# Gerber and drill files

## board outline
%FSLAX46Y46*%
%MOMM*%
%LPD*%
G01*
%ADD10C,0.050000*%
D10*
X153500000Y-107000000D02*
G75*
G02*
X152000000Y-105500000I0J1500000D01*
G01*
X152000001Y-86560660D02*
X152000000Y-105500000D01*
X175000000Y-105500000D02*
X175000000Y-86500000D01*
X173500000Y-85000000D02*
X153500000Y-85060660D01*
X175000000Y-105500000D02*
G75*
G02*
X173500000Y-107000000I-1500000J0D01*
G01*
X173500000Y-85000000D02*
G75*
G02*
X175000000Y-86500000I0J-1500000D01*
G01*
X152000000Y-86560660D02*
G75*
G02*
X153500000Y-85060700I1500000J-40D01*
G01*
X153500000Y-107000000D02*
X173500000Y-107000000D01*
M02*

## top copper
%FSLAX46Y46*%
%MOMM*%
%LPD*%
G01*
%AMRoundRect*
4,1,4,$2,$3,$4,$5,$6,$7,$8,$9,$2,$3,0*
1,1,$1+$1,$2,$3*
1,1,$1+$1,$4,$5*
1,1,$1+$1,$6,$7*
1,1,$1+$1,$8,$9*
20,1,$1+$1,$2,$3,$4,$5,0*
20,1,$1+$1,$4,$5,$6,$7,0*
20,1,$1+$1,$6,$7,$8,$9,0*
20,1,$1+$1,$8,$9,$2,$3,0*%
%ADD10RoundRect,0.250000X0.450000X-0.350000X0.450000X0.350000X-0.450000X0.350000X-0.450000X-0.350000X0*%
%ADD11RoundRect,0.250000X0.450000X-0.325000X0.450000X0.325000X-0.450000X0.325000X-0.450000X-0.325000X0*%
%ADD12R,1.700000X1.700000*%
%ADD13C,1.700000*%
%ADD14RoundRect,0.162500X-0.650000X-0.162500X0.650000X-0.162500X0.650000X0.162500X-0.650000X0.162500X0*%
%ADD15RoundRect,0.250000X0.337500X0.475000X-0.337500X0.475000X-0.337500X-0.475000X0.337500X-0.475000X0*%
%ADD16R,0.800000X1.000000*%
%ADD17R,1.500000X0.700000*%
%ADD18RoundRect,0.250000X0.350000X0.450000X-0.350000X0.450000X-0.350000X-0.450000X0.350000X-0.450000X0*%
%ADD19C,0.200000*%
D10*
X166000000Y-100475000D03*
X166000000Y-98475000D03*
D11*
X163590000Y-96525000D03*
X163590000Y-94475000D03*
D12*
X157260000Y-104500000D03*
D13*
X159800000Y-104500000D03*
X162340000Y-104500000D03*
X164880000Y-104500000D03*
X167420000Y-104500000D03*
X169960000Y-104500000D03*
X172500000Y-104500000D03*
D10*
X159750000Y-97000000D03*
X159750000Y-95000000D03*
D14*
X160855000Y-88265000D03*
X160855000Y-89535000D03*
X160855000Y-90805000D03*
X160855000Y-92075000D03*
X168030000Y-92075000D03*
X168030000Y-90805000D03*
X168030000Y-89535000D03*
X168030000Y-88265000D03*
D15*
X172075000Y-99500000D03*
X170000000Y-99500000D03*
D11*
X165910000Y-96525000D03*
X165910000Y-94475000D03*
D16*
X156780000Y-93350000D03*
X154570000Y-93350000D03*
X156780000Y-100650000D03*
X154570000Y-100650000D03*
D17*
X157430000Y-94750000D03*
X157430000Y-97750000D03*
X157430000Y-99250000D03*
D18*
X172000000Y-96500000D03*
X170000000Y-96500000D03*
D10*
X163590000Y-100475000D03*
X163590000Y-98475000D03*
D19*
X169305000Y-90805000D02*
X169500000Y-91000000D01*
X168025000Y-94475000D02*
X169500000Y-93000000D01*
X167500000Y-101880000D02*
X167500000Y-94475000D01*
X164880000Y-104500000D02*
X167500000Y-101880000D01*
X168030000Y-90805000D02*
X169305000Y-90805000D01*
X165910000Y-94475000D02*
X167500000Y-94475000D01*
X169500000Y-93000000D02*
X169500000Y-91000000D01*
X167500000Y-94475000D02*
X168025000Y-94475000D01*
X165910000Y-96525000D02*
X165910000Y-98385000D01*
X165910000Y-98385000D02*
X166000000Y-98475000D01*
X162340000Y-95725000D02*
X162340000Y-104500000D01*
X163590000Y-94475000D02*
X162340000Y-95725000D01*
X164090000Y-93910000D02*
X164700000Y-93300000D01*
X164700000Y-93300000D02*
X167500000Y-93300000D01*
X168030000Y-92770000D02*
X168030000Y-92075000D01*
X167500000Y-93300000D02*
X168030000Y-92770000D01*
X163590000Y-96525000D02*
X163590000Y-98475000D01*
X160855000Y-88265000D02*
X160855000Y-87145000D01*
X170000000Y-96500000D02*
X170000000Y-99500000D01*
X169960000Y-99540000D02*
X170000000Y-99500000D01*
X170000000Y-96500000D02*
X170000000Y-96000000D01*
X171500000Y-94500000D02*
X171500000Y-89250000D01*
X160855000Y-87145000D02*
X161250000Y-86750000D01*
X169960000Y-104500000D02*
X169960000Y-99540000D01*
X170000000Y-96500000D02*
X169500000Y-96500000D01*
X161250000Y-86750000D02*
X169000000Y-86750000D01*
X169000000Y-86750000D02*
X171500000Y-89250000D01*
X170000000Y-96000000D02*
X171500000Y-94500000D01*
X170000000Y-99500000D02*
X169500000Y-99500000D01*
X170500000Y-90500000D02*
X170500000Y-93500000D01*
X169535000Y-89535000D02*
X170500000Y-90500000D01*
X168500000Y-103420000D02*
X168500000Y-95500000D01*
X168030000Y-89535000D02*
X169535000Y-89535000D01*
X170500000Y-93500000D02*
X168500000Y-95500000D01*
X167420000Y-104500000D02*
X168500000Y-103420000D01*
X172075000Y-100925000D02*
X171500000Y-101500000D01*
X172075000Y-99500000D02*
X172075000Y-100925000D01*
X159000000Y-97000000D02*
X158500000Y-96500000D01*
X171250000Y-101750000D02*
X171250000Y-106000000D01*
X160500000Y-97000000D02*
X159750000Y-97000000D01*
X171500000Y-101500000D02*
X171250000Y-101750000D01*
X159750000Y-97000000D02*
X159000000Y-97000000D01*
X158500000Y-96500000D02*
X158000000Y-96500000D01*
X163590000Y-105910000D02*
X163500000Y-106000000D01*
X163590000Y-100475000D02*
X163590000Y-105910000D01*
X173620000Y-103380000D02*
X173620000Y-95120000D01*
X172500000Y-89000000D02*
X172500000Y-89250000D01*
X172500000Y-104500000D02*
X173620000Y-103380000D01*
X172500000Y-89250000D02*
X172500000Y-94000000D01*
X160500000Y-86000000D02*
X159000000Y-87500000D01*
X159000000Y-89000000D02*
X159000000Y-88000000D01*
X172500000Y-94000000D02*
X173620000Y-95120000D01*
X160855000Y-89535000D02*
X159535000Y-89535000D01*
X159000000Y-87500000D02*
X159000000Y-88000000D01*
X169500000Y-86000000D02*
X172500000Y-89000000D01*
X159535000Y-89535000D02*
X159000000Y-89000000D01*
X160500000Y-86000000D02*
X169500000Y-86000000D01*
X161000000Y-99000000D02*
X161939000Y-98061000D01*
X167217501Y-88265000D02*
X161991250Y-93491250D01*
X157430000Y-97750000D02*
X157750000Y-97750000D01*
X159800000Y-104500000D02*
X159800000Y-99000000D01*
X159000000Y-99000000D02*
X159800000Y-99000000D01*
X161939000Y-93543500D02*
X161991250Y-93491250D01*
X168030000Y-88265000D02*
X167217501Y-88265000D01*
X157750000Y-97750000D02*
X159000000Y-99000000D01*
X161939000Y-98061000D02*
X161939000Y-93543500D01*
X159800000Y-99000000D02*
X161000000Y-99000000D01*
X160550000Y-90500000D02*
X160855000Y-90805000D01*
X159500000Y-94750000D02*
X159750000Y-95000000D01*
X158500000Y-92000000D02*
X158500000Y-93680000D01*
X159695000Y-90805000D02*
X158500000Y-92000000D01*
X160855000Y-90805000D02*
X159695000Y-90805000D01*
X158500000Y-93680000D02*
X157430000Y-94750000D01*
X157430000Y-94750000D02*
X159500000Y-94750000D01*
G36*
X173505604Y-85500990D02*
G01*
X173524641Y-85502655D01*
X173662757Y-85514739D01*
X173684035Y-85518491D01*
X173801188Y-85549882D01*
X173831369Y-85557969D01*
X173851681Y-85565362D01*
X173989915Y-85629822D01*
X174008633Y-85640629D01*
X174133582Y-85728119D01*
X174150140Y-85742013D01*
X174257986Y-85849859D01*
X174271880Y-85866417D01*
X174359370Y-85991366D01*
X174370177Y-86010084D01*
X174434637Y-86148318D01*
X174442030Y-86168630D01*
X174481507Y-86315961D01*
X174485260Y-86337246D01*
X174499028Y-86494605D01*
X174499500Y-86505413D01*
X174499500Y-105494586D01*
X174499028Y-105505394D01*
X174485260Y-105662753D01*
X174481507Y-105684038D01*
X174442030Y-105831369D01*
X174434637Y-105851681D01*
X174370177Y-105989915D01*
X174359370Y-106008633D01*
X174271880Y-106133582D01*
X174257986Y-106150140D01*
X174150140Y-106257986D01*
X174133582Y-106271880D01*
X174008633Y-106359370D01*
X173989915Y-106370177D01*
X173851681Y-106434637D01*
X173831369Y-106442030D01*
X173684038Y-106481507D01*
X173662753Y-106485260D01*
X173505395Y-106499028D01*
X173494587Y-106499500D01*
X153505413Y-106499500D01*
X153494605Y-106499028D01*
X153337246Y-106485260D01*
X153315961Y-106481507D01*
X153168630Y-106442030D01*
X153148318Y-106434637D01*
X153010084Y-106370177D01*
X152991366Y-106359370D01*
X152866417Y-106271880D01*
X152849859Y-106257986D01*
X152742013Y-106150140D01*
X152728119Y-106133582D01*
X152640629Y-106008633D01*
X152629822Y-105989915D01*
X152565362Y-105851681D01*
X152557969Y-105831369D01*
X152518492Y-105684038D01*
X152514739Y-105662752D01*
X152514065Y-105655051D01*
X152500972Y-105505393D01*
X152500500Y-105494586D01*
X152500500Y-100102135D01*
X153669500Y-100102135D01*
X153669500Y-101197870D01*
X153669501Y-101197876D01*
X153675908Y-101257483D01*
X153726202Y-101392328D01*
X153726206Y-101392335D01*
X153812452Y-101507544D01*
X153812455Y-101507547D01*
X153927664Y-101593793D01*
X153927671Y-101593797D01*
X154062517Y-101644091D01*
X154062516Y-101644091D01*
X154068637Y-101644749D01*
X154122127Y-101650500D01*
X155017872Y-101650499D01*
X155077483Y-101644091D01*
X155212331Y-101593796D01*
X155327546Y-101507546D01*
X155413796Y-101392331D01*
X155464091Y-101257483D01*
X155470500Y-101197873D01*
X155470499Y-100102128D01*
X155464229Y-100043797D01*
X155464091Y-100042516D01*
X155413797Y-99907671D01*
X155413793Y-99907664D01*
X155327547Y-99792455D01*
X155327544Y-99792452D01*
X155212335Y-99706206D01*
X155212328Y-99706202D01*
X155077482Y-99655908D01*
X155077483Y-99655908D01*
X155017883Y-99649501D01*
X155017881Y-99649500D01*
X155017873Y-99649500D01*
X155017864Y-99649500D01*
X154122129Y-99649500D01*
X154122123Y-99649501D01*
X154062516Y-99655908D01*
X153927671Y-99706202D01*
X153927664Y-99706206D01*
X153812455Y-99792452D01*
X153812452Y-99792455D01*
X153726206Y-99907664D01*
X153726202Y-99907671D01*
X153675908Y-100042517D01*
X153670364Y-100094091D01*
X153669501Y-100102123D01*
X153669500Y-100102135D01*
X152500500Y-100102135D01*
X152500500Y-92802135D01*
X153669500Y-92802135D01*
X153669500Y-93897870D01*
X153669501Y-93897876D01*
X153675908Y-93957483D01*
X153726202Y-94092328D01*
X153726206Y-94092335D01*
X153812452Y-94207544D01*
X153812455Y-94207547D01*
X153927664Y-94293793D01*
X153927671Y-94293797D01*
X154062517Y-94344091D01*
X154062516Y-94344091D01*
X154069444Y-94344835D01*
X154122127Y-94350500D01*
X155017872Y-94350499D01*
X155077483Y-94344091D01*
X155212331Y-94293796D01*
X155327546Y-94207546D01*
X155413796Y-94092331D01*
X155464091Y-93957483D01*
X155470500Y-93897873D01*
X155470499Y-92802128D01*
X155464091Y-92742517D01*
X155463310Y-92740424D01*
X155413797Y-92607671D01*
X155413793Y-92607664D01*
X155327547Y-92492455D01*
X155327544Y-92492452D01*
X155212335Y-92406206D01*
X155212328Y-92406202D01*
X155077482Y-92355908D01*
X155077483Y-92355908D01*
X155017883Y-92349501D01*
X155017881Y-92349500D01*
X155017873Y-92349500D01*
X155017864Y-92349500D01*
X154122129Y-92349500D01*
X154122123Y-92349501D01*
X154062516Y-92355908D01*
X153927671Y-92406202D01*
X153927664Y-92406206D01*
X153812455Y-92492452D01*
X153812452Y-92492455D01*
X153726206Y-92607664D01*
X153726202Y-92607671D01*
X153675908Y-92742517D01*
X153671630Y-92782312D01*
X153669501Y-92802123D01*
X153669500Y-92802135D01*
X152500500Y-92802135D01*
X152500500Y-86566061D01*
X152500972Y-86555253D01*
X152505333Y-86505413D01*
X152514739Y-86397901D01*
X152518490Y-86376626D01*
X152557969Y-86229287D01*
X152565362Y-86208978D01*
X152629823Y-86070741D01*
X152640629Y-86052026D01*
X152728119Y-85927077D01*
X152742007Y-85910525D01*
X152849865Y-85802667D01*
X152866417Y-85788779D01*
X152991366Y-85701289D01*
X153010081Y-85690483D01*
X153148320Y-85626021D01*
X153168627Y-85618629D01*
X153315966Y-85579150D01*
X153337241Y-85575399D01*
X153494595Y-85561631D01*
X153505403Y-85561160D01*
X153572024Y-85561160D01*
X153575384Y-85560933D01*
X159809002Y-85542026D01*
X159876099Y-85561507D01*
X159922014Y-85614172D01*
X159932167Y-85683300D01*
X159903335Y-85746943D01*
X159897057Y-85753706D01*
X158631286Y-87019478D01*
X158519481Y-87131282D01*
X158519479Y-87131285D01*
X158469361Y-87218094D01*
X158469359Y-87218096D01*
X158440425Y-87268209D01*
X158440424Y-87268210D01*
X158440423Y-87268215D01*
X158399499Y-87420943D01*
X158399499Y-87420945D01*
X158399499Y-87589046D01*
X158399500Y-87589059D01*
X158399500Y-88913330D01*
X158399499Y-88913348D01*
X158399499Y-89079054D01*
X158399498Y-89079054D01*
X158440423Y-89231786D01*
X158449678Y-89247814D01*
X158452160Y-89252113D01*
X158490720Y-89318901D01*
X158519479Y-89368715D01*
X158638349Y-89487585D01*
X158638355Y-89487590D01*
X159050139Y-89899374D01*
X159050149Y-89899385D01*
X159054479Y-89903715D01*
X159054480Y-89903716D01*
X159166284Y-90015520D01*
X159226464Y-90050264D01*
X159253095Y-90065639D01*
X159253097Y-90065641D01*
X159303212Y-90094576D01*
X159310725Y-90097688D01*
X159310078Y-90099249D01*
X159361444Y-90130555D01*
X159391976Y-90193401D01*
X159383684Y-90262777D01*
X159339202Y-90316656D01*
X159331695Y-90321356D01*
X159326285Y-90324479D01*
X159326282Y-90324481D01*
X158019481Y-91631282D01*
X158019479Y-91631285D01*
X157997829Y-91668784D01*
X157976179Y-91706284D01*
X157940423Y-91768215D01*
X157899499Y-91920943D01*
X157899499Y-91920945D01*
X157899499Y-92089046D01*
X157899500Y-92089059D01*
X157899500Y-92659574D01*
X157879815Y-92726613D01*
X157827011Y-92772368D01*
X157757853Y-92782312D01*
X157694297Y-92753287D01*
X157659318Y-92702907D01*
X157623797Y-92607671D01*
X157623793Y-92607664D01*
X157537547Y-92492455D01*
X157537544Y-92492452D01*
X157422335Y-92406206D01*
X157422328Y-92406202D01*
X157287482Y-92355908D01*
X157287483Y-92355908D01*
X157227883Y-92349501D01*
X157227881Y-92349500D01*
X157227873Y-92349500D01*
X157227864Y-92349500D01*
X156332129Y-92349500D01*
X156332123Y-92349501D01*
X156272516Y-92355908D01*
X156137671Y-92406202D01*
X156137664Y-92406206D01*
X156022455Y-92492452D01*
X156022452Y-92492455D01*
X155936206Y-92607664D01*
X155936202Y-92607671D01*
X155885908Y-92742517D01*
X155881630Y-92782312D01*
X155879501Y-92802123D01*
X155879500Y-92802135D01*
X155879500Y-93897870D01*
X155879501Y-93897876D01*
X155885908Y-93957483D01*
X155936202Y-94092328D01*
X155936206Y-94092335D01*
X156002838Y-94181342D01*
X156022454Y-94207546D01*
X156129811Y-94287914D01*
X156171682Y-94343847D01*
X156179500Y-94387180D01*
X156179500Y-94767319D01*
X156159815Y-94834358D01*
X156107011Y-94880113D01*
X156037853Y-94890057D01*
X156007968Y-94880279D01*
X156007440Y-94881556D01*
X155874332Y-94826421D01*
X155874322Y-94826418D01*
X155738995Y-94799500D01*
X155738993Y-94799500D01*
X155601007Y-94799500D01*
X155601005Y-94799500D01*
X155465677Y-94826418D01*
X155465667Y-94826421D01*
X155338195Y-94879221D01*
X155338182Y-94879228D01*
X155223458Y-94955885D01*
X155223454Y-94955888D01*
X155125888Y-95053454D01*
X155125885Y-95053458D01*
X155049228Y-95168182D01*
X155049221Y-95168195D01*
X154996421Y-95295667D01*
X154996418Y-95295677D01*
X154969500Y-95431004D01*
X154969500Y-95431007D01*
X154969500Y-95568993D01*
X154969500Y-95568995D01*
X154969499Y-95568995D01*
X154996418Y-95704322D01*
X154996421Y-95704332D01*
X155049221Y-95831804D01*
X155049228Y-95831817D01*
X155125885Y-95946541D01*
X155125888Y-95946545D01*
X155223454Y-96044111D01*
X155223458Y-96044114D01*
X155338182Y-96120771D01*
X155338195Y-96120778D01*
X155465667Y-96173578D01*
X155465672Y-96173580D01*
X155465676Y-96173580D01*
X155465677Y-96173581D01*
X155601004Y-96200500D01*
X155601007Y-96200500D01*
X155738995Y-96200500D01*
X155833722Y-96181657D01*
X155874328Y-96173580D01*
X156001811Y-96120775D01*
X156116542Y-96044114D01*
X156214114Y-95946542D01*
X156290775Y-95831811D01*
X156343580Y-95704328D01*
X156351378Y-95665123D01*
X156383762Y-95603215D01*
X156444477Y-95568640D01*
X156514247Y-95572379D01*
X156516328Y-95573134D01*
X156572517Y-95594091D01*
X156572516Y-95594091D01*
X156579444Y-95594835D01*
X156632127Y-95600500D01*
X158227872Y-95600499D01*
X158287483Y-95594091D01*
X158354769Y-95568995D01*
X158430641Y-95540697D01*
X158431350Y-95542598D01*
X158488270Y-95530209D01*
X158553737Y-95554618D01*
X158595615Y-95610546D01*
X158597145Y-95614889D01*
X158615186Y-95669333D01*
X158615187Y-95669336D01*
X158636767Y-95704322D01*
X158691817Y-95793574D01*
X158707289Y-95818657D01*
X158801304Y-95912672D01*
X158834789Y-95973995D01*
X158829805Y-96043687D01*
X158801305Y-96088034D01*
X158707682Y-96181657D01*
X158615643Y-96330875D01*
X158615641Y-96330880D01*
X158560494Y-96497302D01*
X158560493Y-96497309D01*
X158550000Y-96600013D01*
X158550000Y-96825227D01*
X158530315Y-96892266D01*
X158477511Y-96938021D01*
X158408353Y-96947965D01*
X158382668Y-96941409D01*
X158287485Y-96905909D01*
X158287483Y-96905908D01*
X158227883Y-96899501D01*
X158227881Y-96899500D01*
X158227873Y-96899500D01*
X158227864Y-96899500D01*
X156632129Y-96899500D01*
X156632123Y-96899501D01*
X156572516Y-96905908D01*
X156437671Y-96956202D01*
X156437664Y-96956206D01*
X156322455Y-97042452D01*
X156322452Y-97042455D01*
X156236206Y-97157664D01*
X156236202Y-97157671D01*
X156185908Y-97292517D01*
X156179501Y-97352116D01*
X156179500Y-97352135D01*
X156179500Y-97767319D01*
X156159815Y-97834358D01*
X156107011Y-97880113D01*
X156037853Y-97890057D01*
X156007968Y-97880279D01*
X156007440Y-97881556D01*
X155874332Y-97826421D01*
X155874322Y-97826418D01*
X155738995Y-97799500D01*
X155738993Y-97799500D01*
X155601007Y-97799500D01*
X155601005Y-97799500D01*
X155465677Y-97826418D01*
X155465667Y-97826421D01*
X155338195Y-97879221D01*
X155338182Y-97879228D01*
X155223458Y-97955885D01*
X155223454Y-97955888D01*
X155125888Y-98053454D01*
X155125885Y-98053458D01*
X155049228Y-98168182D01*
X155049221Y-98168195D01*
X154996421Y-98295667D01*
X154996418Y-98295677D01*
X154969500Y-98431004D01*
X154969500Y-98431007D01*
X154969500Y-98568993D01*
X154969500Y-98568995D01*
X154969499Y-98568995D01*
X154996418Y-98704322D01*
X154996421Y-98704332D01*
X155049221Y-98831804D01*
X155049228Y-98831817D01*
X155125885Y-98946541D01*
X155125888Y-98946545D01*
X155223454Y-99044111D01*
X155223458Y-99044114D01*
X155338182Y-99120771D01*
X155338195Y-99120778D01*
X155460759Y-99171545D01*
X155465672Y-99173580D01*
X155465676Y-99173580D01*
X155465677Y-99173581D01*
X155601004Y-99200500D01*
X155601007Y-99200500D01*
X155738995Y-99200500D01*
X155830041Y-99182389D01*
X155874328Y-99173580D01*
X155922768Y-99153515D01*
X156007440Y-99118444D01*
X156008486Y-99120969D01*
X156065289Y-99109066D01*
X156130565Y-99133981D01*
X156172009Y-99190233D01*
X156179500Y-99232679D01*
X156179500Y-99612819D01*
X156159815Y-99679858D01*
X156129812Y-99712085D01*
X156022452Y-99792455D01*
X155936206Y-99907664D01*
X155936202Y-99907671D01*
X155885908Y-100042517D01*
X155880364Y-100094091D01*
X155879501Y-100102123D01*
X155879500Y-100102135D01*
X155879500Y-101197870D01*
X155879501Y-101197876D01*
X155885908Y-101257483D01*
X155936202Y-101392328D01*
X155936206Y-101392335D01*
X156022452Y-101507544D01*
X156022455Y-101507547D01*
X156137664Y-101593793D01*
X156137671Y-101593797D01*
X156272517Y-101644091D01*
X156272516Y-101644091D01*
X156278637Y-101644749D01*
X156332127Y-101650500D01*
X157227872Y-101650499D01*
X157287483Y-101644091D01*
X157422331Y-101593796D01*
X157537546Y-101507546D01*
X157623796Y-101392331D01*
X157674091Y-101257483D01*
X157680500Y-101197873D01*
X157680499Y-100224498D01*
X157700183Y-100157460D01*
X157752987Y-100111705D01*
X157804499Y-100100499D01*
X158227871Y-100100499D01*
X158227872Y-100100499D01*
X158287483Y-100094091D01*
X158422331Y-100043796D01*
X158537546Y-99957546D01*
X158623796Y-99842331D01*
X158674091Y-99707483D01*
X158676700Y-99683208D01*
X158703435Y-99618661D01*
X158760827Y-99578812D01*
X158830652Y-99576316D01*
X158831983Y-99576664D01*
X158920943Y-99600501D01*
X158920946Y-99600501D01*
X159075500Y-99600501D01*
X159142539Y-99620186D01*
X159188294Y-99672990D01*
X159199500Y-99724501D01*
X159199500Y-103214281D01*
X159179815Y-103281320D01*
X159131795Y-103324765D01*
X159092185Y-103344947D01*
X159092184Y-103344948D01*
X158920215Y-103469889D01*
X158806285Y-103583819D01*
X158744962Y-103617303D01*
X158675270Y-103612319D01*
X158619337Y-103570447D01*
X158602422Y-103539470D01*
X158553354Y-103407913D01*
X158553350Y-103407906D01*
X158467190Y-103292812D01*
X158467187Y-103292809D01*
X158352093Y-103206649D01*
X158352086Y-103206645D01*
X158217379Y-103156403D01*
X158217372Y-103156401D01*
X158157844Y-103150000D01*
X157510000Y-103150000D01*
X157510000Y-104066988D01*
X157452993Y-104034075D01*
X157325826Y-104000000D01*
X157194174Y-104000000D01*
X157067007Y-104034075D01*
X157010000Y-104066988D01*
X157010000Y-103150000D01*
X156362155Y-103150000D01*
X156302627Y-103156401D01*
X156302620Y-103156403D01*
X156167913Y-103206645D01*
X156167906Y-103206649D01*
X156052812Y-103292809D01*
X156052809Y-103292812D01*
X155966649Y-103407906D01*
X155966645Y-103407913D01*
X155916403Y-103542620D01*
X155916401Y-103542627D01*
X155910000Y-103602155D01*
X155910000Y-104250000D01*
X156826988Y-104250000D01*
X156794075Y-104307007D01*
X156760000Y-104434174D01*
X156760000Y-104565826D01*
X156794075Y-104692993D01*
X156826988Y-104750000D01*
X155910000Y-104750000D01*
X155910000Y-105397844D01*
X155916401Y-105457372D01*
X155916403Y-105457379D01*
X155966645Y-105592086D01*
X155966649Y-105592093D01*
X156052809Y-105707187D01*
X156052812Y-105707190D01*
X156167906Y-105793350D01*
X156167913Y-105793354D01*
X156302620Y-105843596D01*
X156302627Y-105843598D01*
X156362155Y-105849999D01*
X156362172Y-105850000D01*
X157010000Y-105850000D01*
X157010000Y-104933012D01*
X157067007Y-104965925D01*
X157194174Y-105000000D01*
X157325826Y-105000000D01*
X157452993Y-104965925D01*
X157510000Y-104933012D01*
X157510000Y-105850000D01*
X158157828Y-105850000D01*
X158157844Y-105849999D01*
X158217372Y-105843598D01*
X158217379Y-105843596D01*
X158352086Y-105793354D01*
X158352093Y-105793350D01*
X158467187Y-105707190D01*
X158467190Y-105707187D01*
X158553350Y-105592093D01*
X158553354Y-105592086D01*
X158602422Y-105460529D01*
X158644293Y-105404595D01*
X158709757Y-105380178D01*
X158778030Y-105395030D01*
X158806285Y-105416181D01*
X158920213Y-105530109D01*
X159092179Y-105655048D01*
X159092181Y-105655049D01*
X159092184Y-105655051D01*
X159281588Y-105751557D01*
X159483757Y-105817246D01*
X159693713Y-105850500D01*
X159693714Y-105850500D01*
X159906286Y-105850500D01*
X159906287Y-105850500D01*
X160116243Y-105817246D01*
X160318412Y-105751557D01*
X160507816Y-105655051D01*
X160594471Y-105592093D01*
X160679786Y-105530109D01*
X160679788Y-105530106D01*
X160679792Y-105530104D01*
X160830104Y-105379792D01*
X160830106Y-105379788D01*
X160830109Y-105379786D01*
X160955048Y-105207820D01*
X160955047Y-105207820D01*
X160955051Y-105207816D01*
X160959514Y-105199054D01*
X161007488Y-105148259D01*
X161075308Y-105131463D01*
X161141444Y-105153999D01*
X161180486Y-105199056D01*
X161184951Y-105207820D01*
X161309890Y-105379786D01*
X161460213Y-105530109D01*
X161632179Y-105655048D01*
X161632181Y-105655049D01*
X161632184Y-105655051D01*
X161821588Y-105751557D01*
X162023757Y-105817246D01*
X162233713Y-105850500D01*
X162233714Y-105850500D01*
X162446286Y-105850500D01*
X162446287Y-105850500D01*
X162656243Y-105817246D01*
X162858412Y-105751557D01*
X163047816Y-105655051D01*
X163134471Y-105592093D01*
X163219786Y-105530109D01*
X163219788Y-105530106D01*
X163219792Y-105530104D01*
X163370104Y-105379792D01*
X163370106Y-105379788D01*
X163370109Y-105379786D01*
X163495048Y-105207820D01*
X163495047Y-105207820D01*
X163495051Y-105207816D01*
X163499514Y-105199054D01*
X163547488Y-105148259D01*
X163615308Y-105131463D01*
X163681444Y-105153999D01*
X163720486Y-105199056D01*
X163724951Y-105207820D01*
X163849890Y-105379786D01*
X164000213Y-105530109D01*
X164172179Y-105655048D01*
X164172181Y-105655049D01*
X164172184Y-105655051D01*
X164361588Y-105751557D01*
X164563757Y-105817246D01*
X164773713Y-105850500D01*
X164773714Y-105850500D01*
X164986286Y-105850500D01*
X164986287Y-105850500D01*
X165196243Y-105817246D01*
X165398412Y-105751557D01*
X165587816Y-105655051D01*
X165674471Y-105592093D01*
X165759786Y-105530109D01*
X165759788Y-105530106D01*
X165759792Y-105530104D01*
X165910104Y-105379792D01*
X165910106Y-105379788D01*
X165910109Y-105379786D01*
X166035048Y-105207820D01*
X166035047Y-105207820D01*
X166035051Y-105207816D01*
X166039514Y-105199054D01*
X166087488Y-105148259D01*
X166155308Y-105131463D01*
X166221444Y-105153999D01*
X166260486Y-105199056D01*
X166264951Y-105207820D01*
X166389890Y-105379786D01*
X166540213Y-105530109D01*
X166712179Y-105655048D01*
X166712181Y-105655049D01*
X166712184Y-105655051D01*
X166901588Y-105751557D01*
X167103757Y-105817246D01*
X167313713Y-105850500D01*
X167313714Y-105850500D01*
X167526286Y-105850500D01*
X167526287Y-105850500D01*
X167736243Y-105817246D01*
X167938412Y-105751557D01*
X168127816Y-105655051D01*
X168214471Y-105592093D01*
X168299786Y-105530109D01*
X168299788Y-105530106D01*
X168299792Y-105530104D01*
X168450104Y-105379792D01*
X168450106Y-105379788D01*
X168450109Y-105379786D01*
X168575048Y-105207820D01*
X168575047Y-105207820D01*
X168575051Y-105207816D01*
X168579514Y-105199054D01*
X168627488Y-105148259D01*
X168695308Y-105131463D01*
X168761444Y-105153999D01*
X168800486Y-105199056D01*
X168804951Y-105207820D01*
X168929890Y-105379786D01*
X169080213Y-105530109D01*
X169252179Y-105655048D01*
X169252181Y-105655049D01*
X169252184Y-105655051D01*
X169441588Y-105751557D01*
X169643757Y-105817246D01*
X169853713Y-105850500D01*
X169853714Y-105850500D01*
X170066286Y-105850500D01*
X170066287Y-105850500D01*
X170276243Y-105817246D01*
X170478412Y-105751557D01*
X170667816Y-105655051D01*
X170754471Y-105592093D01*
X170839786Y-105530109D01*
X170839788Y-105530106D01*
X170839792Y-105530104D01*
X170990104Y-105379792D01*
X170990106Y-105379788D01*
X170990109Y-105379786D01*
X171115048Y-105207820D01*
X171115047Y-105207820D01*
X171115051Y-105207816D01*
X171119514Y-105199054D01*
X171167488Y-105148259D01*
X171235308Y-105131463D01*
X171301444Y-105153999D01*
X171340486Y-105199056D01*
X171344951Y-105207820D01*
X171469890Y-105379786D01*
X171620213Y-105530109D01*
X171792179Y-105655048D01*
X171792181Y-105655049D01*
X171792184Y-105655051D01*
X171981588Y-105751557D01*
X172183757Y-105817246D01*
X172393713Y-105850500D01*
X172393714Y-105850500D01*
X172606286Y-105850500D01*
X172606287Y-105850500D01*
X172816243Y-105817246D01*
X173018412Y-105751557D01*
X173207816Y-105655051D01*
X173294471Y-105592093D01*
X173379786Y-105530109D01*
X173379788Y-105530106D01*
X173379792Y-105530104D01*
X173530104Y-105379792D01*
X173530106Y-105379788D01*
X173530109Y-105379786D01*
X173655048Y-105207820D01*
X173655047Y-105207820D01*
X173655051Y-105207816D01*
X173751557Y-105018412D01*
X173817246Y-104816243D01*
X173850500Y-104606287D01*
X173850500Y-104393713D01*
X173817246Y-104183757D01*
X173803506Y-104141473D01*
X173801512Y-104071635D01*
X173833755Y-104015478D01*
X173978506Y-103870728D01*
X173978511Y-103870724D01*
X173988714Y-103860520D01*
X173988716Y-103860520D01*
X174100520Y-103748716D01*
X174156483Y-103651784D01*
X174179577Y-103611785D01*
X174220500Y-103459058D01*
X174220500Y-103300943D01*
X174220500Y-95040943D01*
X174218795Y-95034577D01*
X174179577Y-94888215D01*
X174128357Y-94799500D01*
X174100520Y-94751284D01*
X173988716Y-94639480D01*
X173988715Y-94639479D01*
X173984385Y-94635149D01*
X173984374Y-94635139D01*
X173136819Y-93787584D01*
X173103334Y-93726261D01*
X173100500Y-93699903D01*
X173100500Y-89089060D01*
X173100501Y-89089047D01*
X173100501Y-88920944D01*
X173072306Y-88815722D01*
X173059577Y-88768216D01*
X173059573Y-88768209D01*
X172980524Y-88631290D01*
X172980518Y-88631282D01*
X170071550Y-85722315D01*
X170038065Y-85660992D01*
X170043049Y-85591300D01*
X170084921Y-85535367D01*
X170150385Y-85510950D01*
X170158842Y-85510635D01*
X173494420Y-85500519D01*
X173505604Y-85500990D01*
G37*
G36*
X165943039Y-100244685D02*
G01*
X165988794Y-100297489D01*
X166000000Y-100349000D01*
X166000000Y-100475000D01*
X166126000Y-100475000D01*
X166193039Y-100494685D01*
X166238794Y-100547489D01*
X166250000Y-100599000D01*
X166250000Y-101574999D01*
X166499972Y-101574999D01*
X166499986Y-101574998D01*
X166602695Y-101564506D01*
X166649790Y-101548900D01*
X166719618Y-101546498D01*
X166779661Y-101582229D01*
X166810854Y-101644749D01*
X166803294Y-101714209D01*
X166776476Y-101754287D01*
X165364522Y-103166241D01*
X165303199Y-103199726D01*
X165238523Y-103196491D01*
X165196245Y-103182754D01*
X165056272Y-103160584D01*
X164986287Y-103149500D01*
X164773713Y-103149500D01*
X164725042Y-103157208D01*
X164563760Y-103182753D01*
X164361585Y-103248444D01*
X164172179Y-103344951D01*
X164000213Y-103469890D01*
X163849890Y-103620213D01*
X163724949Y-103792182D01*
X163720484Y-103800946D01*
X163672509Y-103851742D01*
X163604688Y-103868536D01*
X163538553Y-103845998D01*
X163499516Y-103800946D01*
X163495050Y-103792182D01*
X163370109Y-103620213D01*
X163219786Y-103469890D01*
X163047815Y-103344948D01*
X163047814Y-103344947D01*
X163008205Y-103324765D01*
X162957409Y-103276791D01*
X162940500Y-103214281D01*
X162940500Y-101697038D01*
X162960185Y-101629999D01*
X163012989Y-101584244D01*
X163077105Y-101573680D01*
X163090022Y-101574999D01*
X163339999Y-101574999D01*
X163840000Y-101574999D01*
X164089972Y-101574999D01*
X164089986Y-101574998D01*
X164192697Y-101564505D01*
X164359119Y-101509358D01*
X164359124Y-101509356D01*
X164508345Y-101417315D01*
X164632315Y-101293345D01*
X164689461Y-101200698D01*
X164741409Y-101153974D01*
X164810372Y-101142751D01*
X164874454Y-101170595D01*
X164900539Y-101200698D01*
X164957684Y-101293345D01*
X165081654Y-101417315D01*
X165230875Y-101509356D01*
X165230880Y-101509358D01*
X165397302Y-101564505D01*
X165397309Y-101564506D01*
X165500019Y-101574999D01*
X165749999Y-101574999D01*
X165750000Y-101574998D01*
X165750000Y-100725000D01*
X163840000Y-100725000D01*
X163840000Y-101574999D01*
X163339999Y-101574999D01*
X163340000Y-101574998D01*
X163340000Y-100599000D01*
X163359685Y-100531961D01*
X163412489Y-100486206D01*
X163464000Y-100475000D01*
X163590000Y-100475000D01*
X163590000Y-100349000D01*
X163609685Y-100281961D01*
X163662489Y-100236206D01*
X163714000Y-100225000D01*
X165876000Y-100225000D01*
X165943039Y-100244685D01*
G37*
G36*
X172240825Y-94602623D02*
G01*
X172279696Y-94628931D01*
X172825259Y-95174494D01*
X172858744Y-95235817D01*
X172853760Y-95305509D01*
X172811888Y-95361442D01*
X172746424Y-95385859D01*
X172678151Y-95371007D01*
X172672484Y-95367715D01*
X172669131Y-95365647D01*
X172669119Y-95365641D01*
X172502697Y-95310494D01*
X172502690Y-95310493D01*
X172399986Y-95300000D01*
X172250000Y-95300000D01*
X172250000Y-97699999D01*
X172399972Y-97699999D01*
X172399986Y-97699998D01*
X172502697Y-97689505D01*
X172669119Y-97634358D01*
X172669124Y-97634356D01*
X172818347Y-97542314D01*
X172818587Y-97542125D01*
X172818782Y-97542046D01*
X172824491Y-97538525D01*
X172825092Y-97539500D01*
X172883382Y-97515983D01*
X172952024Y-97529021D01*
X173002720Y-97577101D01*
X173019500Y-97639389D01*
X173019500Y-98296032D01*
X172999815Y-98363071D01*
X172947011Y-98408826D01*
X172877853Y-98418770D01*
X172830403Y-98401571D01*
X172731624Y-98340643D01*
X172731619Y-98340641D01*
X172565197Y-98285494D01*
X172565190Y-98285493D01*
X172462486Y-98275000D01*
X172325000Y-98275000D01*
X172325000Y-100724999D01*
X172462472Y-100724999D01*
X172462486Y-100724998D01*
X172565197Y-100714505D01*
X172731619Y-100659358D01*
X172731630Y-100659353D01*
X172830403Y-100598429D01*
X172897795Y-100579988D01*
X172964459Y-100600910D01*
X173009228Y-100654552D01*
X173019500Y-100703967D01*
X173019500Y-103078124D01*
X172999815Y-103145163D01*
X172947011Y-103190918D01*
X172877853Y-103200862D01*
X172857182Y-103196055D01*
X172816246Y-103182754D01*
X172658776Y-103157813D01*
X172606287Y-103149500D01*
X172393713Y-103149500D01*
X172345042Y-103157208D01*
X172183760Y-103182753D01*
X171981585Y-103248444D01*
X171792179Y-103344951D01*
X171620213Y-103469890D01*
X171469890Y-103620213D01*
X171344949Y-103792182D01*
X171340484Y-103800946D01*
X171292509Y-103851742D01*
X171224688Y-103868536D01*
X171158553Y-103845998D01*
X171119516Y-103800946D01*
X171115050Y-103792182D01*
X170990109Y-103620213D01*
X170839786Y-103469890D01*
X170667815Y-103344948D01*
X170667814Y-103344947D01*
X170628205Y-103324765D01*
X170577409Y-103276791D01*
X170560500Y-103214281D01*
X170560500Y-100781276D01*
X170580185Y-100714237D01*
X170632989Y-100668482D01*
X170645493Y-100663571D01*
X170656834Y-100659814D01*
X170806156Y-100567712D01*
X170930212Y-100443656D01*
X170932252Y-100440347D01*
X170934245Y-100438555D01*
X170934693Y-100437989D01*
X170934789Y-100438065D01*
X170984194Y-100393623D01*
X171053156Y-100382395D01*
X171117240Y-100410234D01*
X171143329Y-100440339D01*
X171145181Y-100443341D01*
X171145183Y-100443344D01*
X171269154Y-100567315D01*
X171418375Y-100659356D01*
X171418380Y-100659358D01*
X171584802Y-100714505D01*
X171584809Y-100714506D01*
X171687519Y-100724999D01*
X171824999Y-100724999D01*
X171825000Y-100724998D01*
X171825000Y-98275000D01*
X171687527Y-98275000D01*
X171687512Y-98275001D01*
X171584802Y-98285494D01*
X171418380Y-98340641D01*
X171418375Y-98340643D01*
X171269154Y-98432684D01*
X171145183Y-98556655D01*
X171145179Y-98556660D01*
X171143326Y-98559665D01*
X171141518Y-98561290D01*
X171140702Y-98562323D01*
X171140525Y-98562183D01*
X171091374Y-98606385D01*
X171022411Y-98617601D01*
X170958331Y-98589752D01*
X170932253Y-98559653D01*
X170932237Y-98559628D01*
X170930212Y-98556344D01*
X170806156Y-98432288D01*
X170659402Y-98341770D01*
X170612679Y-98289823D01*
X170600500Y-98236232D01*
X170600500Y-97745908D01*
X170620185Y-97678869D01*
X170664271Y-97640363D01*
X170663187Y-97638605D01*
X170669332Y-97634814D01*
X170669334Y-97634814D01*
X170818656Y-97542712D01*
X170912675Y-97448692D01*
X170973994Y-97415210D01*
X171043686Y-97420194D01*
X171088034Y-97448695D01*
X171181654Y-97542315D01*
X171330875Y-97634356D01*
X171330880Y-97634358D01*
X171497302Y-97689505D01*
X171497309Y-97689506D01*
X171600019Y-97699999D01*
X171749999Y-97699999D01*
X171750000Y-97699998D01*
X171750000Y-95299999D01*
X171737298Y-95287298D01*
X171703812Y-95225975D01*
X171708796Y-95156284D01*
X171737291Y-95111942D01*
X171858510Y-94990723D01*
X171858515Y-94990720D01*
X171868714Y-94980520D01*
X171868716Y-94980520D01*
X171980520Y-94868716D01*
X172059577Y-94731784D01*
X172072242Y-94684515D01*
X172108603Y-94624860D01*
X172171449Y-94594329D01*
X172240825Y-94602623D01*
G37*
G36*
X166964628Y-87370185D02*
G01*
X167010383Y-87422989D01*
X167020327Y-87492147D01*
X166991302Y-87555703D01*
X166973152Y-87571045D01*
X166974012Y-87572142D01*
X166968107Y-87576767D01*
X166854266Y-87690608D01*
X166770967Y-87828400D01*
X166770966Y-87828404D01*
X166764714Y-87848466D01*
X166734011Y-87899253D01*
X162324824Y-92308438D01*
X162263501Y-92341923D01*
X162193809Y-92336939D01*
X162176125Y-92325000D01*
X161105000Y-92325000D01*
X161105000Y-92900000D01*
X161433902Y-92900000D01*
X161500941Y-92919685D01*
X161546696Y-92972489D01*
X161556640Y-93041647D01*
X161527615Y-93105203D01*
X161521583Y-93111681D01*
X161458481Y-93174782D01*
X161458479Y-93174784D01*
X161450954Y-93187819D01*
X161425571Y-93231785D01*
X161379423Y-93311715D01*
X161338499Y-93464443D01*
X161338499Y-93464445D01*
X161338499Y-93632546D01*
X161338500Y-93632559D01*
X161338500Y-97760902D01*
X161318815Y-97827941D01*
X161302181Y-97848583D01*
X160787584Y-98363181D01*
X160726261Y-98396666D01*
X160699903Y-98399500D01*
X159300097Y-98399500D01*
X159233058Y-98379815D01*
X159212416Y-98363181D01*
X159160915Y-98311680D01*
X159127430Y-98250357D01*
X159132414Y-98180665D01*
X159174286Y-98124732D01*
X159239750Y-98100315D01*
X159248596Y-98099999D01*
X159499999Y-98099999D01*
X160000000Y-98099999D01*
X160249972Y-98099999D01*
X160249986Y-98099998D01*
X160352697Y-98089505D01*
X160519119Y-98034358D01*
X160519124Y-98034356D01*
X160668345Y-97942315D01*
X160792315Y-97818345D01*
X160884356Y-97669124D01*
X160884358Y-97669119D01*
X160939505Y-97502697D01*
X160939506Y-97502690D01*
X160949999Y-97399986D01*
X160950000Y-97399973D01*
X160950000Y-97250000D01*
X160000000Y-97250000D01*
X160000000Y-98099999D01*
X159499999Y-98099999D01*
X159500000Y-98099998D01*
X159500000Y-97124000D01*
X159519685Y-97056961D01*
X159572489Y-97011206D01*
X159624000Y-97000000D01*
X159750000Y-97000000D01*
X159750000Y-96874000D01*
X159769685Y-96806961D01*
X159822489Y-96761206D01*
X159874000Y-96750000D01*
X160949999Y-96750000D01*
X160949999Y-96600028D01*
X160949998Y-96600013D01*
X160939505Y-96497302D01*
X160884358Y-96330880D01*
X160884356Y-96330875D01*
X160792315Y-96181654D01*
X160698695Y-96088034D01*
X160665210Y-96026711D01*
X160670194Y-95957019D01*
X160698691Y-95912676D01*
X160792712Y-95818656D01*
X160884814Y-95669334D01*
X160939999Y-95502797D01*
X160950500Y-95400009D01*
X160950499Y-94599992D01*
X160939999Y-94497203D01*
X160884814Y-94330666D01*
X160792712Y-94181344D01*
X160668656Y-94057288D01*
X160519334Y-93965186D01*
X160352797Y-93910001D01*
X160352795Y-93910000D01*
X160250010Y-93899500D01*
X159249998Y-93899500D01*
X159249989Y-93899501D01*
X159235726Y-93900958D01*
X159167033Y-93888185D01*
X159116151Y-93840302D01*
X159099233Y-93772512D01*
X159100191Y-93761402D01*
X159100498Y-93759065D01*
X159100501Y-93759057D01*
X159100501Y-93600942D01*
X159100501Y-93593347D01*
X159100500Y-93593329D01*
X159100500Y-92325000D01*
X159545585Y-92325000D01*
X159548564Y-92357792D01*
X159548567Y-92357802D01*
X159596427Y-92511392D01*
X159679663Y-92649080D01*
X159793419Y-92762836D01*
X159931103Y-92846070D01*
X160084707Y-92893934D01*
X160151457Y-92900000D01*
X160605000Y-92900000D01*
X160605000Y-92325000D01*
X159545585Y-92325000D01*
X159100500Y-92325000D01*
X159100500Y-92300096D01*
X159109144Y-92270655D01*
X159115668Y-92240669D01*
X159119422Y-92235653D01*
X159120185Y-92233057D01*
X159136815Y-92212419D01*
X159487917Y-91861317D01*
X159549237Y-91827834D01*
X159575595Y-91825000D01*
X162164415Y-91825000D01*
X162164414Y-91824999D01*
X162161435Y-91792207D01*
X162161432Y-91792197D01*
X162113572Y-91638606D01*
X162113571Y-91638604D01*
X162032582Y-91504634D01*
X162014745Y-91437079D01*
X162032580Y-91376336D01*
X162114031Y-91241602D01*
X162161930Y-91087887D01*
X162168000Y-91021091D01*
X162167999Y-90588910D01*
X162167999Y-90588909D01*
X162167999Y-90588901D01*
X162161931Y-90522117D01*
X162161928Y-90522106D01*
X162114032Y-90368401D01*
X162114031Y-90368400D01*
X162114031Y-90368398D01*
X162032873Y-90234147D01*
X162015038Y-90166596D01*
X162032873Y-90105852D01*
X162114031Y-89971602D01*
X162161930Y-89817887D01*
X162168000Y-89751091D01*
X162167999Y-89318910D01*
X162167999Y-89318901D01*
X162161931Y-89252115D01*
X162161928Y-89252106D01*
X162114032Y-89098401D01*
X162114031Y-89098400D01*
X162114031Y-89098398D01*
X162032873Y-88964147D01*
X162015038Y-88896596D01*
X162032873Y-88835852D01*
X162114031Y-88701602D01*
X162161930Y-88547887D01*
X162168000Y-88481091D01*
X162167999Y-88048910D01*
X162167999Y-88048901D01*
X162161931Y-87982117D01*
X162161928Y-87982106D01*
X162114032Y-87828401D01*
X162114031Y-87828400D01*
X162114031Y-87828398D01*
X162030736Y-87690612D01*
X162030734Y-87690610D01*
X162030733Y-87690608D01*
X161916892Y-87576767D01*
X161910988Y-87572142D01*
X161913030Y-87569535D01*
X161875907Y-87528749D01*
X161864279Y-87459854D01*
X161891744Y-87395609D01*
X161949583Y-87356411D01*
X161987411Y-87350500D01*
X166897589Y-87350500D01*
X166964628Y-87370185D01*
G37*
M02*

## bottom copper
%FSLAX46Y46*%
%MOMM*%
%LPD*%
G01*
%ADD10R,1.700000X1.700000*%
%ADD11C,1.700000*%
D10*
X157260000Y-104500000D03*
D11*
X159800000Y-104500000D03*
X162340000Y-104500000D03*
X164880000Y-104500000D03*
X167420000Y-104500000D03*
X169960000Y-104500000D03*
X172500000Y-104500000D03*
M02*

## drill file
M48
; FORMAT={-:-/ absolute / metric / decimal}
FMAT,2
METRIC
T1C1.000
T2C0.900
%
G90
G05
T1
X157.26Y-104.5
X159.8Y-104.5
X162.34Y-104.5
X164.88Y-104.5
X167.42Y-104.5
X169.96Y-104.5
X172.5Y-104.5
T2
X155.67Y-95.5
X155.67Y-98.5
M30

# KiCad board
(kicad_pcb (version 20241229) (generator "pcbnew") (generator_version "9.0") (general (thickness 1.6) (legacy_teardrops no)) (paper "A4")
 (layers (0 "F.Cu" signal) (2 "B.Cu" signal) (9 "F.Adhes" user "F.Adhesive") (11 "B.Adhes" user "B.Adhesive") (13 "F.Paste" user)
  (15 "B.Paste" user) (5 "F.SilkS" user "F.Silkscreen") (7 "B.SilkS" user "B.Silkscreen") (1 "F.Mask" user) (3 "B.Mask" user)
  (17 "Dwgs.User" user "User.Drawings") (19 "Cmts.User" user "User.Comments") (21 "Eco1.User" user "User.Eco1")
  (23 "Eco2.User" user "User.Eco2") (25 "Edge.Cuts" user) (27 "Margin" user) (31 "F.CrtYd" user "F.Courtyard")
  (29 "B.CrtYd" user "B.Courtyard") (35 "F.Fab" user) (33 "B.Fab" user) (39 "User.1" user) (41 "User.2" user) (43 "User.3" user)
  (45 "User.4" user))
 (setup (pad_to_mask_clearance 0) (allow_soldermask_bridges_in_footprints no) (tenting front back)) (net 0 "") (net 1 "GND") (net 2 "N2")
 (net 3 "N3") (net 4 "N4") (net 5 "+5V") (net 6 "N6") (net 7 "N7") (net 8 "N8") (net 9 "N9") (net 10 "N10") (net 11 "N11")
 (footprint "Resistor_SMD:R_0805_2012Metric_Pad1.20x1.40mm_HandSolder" (layer "F.Cu") (at 166 99.475 90)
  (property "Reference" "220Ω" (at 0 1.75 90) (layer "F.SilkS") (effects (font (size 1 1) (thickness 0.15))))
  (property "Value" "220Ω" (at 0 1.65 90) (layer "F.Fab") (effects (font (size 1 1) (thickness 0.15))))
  (pad "1" smd roundrect (at -1 0 90) (size 1.2 1.4) (layers "F.Cu" "F.Mask" "F.Paste") (roundrect_rratio 0.208333) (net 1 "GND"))
  (pad "2" smd roundrect (at 1 0 90) (size 1.2 1.4) (layers "F.Cu" "F.Mask" "F.Paste") (roundrect_rratio 0.208333) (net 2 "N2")))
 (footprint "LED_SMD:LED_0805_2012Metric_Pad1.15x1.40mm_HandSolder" (layer "F.Cu") (at 163.59 95.5 90)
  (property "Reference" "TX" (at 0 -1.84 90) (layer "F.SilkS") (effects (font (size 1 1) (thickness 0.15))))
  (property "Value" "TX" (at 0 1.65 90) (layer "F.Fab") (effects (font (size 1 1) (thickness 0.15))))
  (pad "1" smd roundrect (at -1.025 0 90) (size 1.15 1.4) (layers "F.Cu" "F.Mask" "F.Paste") (roundrect_rratio 0.217391) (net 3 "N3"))
  (pad "2" smd roundrect (at 1.025 0 90) (size 1.15 1.4) (layers "F.Cu" "F.Mask" "F.Paste") (roundrect_rratio 0.217391) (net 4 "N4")))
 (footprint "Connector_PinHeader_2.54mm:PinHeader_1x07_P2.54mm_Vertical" (layer "F.Cu") (at 157.26 104.5 90)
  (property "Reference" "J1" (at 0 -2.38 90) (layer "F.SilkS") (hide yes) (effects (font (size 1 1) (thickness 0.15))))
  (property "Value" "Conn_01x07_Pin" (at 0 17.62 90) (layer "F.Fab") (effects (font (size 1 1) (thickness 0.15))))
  (pad "1" thru_hole rect (at 0 0 90) (size 1.7 1.7) (drill 1) (layers "*.Cu" "*.Mask") (remove_unused_layers no) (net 1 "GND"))
  (pad "2" thru_hole circle (at 0 2.54 90) (size 1.7 1.7) (drill 1) (layers "*.Cu" "*.Mask") (remove_unused_layers no) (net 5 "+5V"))
  (pad "3" thru_hole circle (at 0 5.08 90) (size 1.7 1.7) (drill 1) (layers "*.Cu" "*.Mask") (remove_unused_layers no) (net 4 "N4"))
  (pad "4" thru_hole circle (at 0 7.62 90) (size 1.7 1.7) (drill 1) (layers "*.Cu" "*.Mask") (remove_unused_layers no) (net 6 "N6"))
  (pad "5" thru_hole circle (at 0 10.16 90) (size 1.7 1.7) (drill 1) (layers "*.Cu" "*.Mask") (remove_unused_layers no) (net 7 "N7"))
  (pad "6" thru_hole circle (at 0 12.7 90) (size 1.7 1.7) (drill 1) (layers "*.Cu" "*.Mask") (remove_unused_layers no) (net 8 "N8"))
  (pad "7" thru_hole circle (at 0 15.24 90) (size 1.7 1.7) (drill 1) (layers "*.Cu" "*.Mask") (remove_unused_layers no) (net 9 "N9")))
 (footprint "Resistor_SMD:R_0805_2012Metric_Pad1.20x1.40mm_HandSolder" (layer "F.Cu") (at 159.75 96 90)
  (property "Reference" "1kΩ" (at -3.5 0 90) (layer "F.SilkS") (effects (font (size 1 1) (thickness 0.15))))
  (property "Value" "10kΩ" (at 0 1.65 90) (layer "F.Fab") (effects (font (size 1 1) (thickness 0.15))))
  (pad "1" smd roundrect (at -1 0 90) (size 1.2 1.4) (layers "F.Cu" "F.Mask" "F.Paste") (roundrect_rratio 0.208333) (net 1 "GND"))
  (pad "2" smd roundrect (at 1 0 90) (size 1.2 1.4) (layers "F.Cu" "F.Mask" "F.Paste") (roundrect_rratio 0.208333) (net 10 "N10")))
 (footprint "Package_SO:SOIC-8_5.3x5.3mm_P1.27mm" (layer "F.Cu") (at 164.4425 90.17)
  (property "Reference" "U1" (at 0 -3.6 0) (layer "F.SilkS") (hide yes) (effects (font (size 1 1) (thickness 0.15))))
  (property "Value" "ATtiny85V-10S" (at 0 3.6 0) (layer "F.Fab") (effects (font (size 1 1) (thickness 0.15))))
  (pad "1" smd roundrect (at -3.5875 -1.905) (size 1.625 0.65) (layers "F.Cu" "F.Mask" "F.Paste") (roundrect_rratio 0.25) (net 8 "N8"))
  (pad "2" smd roundrect (at -3.5875 -0.635) (size 1.625 0.65) (layers "F.Cu" "F.Mask" "F.Paste") (roundrect_rratio 0.25) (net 9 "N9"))
  (pad "3" smd roundrect (at -3.5875 0.635) (size 1.625 0.65) (layers "F.Cu" "F.Mask" "F.Paste") (roundrect_rratio 0.25) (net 10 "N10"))
  (pad "4" smd roundrect (at -3.5875 1.905) (size 1.625 0.65) (layers "F.Cu" "F.Mask" "F.Paste") (roundrect_rratio 0.25) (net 1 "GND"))
  (pad "5" smd roundrect (at 3.5875 1.905) (size 1.625 0.65) (layers "F.Cu" "F.Mask" "F.Paste") (roundrect_rratio 0.25) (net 4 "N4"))
  (pad "6" smd roundrect (at 3.5875 0.635) (size 1.625 0.65) (layers "F.Cu" "F.Mask" "F.Paste") (roundrect_rratio 0.25) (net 6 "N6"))
  (pad "7" smd roundrect (at 3.5875 -0.635) (size 1.625 0.65) (layers "F.Cu" "F.Mask" "F.Paste") (roundrect_rratio 0.25) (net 7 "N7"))
  (pad "8" smd roundrect (at 3.5875 -1.905) (size 1.625 0.65) (layers "F.Cu" "F.Mask" "F.Paste") (roundrect_rratio 0.25) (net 5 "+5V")))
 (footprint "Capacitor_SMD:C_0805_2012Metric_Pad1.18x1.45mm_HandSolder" (layer "F.Cu") (at 171.0375 99.5 180)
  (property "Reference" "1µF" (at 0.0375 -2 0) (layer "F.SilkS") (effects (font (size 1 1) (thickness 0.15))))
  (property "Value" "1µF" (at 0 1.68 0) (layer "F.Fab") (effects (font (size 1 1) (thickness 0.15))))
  (pad "1" smd roundrect (at -1.0375 0 180) (size 1.175 1.45) (layers "F.Cu" "F.Mask" "F.Paste") (roundrect_rratio 0.212766) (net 1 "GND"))
  (pad "2" smd roundrect (at 1.0375 0 180) (size 1.175 1.45) (layers "F.Cu" "F.Mask" "F.Paste") (roundrect_rratio 0.212766) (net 8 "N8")))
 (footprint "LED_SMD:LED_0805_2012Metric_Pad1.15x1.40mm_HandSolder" (layer "F.Cu") (at 165.91 95.5 90)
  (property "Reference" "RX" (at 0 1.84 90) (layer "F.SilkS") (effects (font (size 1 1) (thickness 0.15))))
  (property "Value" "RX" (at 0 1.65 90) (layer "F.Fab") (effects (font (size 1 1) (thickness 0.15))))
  (pad "1" smd roundrect (at -1.025 0 90) (size 1.15 1.4) (layers "F.Cu" "F.Mask" "F.Paste") (roundrect_rratio 0.217391) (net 2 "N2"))
  (pad "2" smd roundrect (at 1.025 0 90) (size 1.15 1.4) (layers "F.Cu" "F.Mask" "F.Paste") (roundrect_rratio 0.217391) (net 6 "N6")))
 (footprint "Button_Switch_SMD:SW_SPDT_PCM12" (layer "F.Cu") (at 156 97 -90)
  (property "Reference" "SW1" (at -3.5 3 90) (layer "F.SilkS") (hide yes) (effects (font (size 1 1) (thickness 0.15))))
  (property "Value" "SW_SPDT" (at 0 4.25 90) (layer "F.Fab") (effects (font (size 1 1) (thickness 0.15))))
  (pad "" smd rect (at -3.65 -0.78 270) (size 1 0.8) (layers "F.Cu" "F.Mask" "F.Paste"))
  (pad "" smd rect (at -3.65 1.43 270) (size 1 0.8) (layers "F.Cu" "F.Mask" "F.Paste"))
  (pad "" np_thru_hole circle (at -1.5 0.33 270) (size 0.9 0.9) (drill 0.9) (layers "*.Cu" "*.Mask"))
  (pad "" np_thru_hole circle (at 1.5 0.33 270) (size 0.9 0.9) (drill 0.9) (layers "*.Cu" "*.Mask"))
  (pad "" smd rect (at 3.65 -0.78 270) (size 1 0.8) (layers "F.Cu" "F.Mask" "F.Paste"))
  (pad "" smd rect (at 3.65 1.43 270) (size 1 0.8) (layers "F.Cu" "F.Mask" "F.Paste"))
  (pad "1" smd rect (at -2.25 -1.43 270) (size 0.7 1.5) (layers "F.Cu" "F.Mask" "F.Paste") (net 10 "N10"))
  (pad "2" smd rect (at 0.75 -1.43 270) (size 0.7 1.5) (layers "F.Cu" "F.Mask" "F.Paste") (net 5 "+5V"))
  (pad "3" smd rect (at 2.25 -1.43 270) (size 0.7 1.5) (layers "F.Cu" "F.Mask" "F.Paste") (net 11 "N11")))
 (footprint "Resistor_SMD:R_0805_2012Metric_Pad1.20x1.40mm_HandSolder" (layer "F.Cu") (at 171 96.5 180)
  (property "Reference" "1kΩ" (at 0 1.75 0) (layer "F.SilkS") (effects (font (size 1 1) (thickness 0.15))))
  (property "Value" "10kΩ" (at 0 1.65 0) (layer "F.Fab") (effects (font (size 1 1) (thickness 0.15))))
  (pad "1" smd roundrect (at -1 0 180) (size 1.2 1.4) (layers "F.Cu" "F.Mask" "F.Paste") (roundrect_rratio 0.208333) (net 1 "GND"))
  (pad "2" smd roundrect (at 1 0 180) (size 1.2 1.4) (layers "F.Cu" "F.Mask" "F.Paste") (roundrect_rratio 0.208333) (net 8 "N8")))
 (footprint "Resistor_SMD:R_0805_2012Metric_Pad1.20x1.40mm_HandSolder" (layer "F.Cu") (at 163.59 99.475 90)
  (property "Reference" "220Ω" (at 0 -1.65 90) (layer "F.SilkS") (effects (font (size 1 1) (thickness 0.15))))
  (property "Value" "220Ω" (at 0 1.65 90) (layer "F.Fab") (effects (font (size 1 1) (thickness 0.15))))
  (pad "1" smd roundrect (at -1 0 90) (size 1.2 1.4) (layers "F.Cu" "F.Mask" "F.Paste") (roundrect_rratio 0.208333) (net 1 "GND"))
  (pad "2" smd roundrect (at 1 0 90) (size 1.2 1.4) (layers "F.Cu" "F.Mask" "F.Paste") (roundrect_rratio 0.208333) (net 3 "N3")))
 (gr_arc (start 153.5 107) (mid 152.43934 106.56066) (end 152 105.5) (stroke (width 0.05) (type default)) (layer "Edge.Cuts"))
 (gr_line (start 152.000001 86.56066) (end 152 105.5) (stroke (width 0.05) (type default)) (layer "Edge.Cuts"))
 (gr_line (start 175 105.5) (end 175 86.5) (stroke (width 0.05) (type default)) (layer "Edge.Cuts"))
 (gr_line (start 173.5 85) (end 153.5 85.06066) (stroke (width 0.05) (type default)) (layer "Edge.Cuts"))
 (gr_arc (start 175 105.5) (mid 174.56066 106.56066) (end 173.5 107) (stroke (width 0.05) (type default)) (layer "Edge.Cuts"))
 (gr_arc (start 173.5 85) (mid 174.56066 85.43934) (end 175 86.5) (stroke (width 0.05) (type default)) (layer "Edge.Cuts"))
 (gr_arc (start 152 86.56066) (mid 152.43934 85.5) (end 153.5 85.06066) (stroke (width 0.05) (type default)) (layer "Edge.Cuts"))
 (gr_line (start 153.5 107) (end 173.5 107) (stroke (width 0.05) (type default)) (layer "Edge.Cuts"))
 (segment (start 169.305 90.805) (end 169.5 91) (width 0.2) (layer "F.Cu") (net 6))
 (segment (start 168.025 94.475) (end 169.5 93) (width 0.2) (layer "F.Cu") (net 6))
 (segment (start 167.5 101.88) (end 167.5 94.475) (width 0.2) (layer "F.Cu") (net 6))
 (segment (start 164.88 104.5) (end 167.5 101.88) (width 0.2) (layer "F.Cu") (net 6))
 (segment (start 168.03 90.805) (end 169.305 90.805) (width 0.2) (layer "F.Cu") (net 6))
 (segment (start 165.91 94.475) (end 167.5 94.475) (width 0.2) (layer "F.Cu") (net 6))
 (segment (start 169.5 93) (end 169.5 91) (width 0.2) (layer "F.Cu") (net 6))
 (segment (start 167.5 94.475) (end 168.025 94.475) (width 0.2) (layer "F.Cu") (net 6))
 (segment (start 165.91 96.525) (end 165.91 98.385) (width 0.2) (layer "F.Cu") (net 2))
 (segment (start 165.91 98.385) (end 166 98.475) (width 0.2) (layer "F.Cu") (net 2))
 (segment (start 162.34 95.725) (end 162.34 104.5) (width 0.2) (layer "F.Cu") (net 4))
 (segment (start 163.59 94.475) (end 162.34 95.725) (width 0.2) (layer "F.Cu") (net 4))
 (segment (start 164.09 93.91) (end 164.7 93.3) (width 0.2) (layer "F.Cu") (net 4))
 (segment (start 164.7 93.3) (end 167.5 93.3) (width 0.2) (layer "F.Cu") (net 4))
 (segment (start 168.03 92.77) (end 168.03 92.075) (width 0.2) (layer "F.Cu") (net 4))
 (segment (start 167.5 93.3) (end 168.03 92.77) (width 0.2) (layer "F.Cu") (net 4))
 (segment (start 163.59 96.525) (end 163.59 98.475) (width 0.2) (layer "F.Cu") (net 3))
 (segment (start 160.855 88.265) (end 160.855 87.145) (width 0.2) (layer "F.Cu") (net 8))
 (segment (start 170 96.5) (end 170 99.5) (width 0.2) (layer "F.Cu") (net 8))
 (segment (start 169.96 99.54) (end 170 99.5) (width 0.2) (layer "F.Cu") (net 8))
 (segment (start 170 96.5) (end 170 96) (width 0.2) (layer "F.Cu") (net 8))
 (segment (start 171.5 94.5) (end 171.5 89.25) (width 0.2) (layer "F.Cu") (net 8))
 (segment (start 160.855 87.145) (end 161.25 86.75) (width 0.2) (layer "F.Cu") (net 8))
 (segment (start 169.96 104.5) (end 169.96 99.54) (width 0.2) (layer "F.Cu") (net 8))
 (segment (start 170 96.5) (end 169.5 96.5) (width 0.2) (layer "F.Cu") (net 8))
 (segment (start 161.25 86.75) (end 169 86.75) (width 0.2) (layer "F.Cu") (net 8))
 (segment (start 169 86.75) (end 171.5 89.25) (width 0.2) (layer "F.Cu") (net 8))
 (segment (start 170 96) (end 171.5 94.5) (width 0.2) (layer "F.Cu") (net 8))
 (segment (start 170 99.5) (end 169.5 99.5) (width 0.2) (layer "F.Cu") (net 8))
 (segment (start 170.5 90.5) (end 170.5 93.5) (width 0.2) (layer "F.Cu") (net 7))
 (segment (start 169.535 89.535) (end 170.5 90.5) (width 0.2) (layer "F.Cu") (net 7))
 (segment (start 168.5 103.42) (end 168.5 95.5) (width 0.2) (layer "F.Cu") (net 7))
 (segment (start 168.03 89.535) (end 169.535 89.535) (width 0.2) (layer "F.Cu") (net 7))
 (segment (start 170.5 93.5) (end 168.5 95.5) (width 0.2) (layer "F.Cu") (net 7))
 (segment (start 167.42 104.5) (end 168.5 103.42) (width 0.2) (layer "F.Cu") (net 7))
 (segment (start 172.075 100.925) (end 171.5 101.5) (width 0.2) (layer "F.Cu") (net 1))
 (segment (start 172.075 99.5) (end 172.075 100.925) (width 0.2) (layer "F.Cu") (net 1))
 (segment (start 159 97) (end 158.5 96.5) (width 0.2) (layer "F.Cu") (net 1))
 (segment (start 171.25 101.75) (end 171.25 106) (width 0.2) (layer "F.Cu") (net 1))
 (segment (start 160.5 97) (end 159.75 97) (width 0.2) (layer "F.Cu") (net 1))
 (segment (start 171.5 101.5) (end 171.25 101.75) (width 0.2) (layer "F.Cu") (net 1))
 (segment (start 159.75 97) (end 159 97) (width 0.2) (layer "F.Cu") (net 1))
 (segment (start 158.5 96.5) (end 158 96.5) (width 0.2) (layer "F.Cu") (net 1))
 (segment (start 163.59 105.91) (end 163.5 106) (width 0.2) (layer "F.Cu") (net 1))
 (segment (start 163.59 100.475) (end 163.59 105.91) (width 0.2) (layer "F.Cu") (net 1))
 (segment (start 173.62 103.38) (end 173.62 95.12) (width 0.2) (layer "F.Cu") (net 9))
 (segment (start 172.5 89) (end 172.5 89.25) (width 0.2) (layer "F.Cu") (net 9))
 (segment (start 172.5 104.5) (end 173.62 103.38) (width 0.2) (layer "F.Cu") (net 9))
 (segment (start 172.5 89.25) (end 172.5 94) (width 0.2) (layer "F.Cu") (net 9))
 (segment (start 160.5 86) (end 159 87.5) (width 0.2) (layer "F.Cu") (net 9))
 (segment (start 159 89) (end 159 88) (width 0.2) (layer "F.Cu") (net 9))
 (segment (start 172.5 94) (end 173.62 95.12) (width 0.2) (layer "F.Cu") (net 9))
 (segment (start 160.855 89.535) (end 159.535 89.535) (width 0.2) (layer "F.Cu") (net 9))
 (segment (start 159 87.5) (end 159 88) (width 0.2) (layer "F.Cu") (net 9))
 (segment (start 169.5 86) (end 172.5 89) (width 0.2) (layer "F.Cu") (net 9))
 (segment (start 159.535 89.535) (end 159 89) (width 0.2) (layer "F.Cu") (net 9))
 (segment (start 160.5 86) (end 169.5 86) (width 0.2) (layer "F.Cu") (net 9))
 (segment (start 161 99) (end 161.939 98.061) (width 0.2) (layer "F.Cu") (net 5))
 (segment (start 167.217501 88.265) (end 161.99125 93.49125) (width 0.2) (layer "F.Cu") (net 5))
 (segment (start 157.43 97.75) (end 157.75 97.75) (width 0.2) (layer "F.Cu") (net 5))
 (segment (start 159.8 104.5) (end 159.8 99) (width 0.2) (layer "F.Cu") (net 5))
 (segment (start 159 99) (end 159.8 99) (width 0.2) (layer "F.Cu") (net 5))
 (segment (start 161.939 93.5435) (end 161.99125 93.49125) (width 0.2) (layer "F.Cu") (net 5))
 (segment (start 168.03 88.265) (end 167.217501 88.265) (width 0.2) (layer "F.Cu") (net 5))
 (segment (start 157.75 97.75) (end 159 99) (width 0.2) (layer "F.Cu") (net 5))
 (segment (start 161.939 98.061) (end 161.939 93.5435) (width 0.2) (layer "F.Cu") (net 5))
 (segment (start 159.8 99) (end 161 99) (width 0.2) (layer "F.Cu") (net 5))
 (segment (start 160.55 90.5) (end 160.855 90.805) (width 0.2) (layer "F.Cu") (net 10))
 (segment (start 159.5 94.75) (end 159.75 95) (width 0.2) (layer "F.Cu") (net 10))
 (segment (start 158.5 92) (end 158.5 93.68) (width 0.2) (layer "F.Cu") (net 10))
 (segment (start 159.695 90.805) (end 158.5 92) (width 0.2) (layer "F.Cu") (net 10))
 (segment (start 160.855 90.805) (end 159.695 90.805) (width 0.2) (layer "F.Cu") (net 10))
 (segment (start 158.5 93.68) (end 157.43 94.75) (width 0.2) (layer "F.Cu") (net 10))
 (segment (start 157.43 94.75) (end 159.5 94.75) (width 0.2) (layer "F.Cu") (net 10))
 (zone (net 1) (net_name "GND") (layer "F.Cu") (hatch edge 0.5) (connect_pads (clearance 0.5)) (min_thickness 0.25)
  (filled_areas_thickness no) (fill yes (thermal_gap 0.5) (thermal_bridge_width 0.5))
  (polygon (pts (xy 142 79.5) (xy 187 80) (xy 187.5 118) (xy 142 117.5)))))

